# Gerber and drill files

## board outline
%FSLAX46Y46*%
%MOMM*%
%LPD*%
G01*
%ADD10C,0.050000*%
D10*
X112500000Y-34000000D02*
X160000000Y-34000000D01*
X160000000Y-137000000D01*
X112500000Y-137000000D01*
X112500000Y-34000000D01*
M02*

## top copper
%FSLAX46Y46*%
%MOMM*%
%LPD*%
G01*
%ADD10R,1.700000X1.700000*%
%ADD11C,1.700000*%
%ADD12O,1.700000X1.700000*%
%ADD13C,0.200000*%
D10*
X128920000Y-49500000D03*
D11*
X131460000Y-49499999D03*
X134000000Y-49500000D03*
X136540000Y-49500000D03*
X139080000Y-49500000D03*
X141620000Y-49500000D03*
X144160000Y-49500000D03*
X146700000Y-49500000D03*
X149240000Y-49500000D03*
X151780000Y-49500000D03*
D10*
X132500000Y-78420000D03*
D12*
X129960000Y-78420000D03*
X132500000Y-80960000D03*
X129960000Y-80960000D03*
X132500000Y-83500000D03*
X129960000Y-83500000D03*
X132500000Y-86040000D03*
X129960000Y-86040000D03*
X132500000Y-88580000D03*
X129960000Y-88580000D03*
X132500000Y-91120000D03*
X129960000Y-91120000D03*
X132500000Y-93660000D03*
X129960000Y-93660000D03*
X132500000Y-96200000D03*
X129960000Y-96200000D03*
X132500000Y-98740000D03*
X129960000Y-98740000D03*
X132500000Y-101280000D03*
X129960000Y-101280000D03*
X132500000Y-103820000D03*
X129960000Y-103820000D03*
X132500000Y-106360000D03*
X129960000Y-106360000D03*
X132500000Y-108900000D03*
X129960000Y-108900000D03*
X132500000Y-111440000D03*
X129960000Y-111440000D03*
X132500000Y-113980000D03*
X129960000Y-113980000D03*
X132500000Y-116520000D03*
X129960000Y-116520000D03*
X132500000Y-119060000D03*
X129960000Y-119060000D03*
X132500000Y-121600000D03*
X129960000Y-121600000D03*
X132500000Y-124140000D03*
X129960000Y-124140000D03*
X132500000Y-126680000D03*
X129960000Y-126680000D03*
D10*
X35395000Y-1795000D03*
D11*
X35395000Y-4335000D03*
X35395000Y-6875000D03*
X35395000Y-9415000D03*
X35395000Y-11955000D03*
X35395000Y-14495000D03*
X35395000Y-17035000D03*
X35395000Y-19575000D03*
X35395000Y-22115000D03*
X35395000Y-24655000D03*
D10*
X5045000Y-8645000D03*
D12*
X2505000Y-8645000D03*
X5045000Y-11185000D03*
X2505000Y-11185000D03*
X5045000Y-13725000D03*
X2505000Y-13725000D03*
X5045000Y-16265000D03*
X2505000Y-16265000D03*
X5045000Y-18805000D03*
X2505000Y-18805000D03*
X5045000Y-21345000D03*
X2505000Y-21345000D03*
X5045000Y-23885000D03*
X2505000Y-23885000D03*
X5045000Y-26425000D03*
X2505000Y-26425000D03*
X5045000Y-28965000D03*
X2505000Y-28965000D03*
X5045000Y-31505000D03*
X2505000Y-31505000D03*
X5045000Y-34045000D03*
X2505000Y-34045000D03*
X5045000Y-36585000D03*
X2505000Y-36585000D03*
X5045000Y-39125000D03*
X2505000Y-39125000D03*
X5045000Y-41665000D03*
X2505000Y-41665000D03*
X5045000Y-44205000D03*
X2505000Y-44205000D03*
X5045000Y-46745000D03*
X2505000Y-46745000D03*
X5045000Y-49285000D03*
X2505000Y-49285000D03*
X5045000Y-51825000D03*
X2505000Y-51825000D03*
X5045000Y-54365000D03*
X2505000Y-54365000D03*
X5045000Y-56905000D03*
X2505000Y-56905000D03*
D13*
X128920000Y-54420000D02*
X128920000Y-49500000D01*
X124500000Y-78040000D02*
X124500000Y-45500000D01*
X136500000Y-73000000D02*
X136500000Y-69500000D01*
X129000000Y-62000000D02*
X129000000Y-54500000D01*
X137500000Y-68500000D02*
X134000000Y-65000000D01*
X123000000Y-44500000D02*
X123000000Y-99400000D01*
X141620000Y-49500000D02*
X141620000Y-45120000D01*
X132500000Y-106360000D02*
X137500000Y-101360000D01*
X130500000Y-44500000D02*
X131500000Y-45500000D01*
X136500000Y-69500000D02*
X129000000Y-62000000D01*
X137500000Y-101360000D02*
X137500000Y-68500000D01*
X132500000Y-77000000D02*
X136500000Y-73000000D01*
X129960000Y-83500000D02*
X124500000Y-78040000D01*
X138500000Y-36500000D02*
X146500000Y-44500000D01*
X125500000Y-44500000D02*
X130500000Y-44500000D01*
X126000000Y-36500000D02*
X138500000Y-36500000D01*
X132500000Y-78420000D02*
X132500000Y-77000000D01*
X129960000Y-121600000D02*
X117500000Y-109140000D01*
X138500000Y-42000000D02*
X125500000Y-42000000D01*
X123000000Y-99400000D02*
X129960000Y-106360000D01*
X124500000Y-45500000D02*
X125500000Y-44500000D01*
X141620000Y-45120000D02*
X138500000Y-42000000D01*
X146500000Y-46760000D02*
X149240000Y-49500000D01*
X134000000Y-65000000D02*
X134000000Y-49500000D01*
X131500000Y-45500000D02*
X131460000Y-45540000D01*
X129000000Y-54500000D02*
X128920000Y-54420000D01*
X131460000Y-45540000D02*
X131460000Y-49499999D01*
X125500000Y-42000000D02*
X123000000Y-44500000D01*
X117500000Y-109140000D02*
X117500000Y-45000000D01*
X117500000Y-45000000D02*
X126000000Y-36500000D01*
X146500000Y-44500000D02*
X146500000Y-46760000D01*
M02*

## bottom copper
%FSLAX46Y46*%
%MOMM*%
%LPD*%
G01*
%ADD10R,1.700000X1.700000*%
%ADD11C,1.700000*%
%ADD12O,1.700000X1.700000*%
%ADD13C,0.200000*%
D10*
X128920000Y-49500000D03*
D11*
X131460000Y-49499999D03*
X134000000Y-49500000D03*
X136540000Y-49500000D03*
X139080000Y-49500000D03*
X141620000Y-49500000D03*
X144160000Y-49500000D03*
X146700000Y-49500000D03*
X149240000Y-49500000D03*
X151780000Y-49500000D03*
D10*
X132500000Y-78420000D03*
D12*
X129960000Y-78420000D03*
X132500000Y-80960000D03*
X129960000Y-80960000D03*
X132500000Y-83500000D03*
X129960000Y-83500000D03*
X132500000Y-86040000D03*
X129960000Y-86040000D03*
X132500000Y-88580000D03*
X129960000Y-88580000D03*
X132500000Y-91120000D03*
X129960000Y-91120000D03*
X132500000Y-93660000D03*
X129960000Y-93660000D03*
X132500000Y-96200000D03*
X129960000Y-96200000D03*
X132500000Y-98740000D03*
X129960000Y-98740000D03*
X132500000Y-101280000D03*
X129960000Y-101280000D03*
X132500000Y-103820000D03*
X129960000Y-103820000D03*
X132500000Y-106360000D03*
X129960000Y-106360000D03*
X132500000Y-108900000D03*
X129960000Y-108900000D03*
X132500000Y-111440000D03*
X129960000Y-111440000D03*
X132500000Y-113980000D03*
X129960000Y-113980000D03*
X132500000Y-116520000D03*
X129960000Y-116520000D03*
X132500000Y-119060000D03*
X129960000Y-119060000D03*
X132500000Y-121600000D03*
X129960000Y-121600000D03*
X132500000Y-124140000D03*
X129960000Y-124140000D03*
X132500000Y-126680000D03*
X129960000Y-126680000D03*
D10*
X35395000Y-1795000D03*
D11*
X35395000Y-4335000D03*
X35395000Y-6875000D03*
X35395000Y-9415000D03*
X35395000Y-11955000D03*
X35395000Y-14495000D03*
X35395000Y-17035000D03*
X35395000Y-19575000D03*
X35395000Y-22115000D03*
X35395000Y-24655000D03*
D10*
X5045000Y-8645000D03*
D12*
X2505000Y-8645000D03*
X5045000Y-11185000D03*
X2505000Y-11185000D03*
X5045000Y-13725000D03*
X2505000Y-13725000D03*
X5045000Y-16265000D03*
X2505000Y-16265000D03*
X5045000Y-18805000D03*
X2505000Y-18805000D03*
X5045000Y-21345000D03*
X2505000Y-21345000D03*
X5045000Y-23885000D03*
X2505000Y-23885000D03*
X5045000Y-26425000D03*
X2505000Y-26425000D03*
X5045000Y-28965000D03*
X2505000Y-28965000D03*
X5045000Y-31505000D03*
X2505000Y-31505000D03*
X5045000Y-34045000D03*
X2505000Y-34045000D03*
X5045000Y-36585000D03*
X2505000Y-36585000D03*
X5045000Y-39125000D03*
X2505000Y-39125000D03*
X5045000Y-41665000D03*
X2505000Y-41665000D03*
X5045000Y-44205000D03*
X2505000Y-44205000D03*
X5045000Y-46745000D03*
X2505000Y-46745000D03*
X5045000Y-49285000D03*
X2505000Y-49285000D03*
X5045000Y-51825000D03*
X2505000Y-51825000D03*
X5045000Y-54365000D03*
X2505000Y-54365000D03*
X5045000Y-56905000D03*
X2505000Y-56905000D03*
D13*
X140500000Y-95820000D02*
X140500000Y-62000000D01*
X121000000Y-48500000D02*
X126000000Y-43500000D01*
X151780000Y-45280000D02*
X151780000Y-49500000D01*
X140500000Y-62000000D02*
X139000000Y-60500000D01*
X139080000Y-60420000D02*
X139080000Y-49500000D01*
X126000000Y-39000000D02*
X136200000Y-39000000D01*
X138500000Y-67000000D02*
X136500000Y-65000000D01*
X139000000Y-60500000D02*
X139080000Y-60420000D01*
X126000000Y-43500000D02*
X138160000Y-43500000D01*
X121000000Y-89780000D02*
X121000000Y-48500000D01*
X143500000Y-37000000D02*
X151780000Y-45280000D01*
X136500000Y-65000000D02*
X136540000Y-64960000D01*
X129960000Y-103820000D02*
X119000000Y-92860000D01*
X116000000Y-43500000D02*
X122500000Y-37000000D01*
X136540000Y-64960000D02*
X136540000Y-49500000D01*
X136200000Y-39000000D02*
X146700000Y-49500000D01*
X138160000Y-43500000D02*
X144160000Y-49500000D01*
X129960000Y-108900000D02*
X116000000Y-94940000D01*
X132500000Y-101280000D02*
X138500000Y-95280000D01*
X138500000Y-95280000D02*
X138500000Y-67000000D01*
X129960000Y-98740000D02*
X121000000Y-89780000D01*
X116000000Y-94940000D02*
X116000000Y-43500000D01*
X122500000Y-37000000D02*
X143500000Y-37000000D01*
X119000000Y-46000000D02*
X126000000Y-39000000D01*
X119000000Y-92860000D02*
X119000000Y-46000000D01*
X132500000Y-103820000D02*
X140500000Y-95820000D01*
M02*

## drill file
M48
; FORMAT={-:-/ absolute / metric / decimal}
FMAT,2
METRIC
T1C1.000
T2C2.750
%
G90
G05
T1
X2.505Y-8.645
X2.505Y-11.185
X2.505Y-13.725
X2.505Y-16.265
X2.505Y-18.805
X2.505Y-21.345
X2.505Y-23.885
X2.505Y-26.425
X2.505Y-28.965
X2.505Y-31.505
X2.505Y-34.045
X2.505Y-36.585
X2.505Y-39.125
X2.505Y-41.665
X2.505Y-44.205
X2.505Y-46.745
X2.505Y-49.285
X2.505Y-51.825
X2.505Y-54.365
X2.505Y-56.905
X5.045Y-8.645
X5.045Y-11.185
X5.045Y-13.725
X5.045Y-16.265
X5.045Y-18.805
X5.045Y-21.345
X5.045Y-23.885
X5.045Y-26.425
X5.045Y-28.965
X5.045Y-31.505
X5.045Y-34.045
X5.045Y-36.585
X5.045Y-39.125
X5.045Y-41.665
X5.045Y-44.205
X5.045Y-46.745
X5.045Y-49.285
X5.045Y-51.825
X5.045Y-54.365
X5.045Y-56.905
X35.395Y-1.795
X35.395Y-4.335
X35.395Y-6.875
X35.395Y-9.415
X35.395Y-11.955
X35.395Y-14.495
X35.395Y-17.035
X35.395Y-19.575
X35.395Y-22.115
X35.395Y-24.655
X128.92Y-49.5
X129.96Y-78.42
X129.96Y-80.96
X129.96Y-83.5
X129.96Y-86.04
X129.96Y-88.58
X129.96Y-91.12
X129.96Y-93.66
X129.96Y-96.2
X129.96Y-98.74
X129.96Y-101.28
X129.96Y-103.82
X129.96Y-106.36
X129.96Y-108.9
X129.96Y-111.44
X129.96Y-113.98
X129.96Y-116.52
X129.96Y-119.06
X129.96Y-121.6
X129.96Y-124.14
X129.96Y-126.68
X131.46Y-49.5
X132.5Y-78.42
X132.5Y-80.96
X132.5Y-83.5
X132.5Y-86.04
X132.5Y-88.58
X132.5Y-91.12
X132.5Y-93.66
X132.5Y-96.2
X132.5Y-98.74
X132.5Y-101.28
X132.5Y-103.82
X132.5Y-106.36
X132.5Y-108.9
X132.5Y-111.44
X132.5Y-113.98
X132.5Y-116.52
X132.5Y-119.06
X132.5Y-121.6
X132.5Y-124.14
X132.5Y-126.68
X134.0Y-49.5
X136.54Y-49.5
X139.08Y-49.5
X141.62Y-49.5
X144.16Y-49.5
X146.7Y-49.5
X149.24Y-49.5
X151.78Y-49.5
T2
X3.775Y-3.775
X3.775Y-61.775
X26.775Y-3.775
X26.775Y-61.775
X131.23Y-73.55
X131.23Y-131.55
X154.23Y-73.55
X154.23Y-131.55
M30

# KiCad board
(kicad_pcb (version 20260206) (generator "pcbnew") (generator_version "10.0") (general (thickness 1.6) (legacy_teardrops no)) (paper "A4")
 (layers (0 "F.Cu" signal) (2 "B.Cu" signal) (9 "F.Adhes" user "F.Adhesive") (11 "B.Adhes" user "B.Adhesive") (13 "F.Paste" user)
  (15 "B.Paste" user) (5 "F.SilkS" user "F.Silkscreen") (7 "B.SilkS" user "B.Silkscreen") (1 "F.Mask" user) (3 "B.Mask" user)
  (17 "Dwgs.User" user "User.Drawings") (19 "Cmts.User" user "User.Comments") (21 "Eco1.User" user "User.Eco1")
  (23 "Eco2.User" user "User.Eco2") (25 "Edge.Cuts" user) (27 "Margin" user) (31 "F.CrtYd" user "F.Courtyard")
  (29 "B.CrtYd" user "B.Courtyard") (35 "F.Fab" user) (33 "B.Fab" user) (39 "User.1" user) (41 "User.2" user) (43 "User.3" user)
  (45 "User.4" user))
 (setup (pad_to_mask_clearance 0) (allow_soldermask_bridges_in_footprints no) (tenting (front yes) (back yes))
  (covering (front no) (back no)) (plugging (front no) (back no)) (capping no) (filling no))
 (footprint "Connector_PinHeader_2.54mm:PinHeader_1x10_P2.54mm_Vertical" (layer "F.Cu") (at 128.92 49.5 90)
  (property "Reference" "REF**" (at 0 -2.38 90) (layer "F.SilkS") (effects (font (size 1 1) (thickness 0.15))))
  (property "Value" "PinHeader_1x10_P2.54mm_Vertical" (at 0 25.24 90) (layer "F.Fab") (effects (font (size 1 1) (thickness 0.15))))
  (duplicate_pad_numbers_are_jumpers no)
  (pad "1" thru_hole rect (at 0 0 90) (size 1.7 1.7) (drill 1) (layers "*.Cu" "*.Mask") (remove_unused_layers no))
  (pad "2" thru_hole circle (at 0.000001 2.54 90) (size 1.7 1.7) (drill 1) (layers "*.Cu" "*.Mask") (remove_unused_layers no))
  (pad "3" thru_hole circle (at 0 5.08 90) (size 1.7 1.7) (drill 1) (layers "*.Cu" "*.Mask") (remove_unused_layers no))
  (pad "4" thru_hole circle (at 0 7.62 90) (size 1.7 1.7) (drill 1) (layers "*.Cu" "*.Mask") (remove_unused_layers no))
  (pad "5" thru_hole circle (at 0 10.16 90) (size 1.7 1.7) (drill 1) (layers "*.Cu" "*.Mask") (remove_unused_layers no))
  (pad "6" thru_hole circle (at 0 12.7 90) (size 1.7 1.7) (drill 1) (layers "*.Cu" "*.Mask") (remove_unused_layers no))
  (pad "7" thru_hole circle (at 0 15.24 90) (size 1.7 1.7) (drill 1) (layers "*.Cu" "*.Mask") (remove_unused_layers no))
  (pad "8" thru_hole circle (at 0 17.78 90) (size 1.7 1.7) (drill 1) (layers "*.Cu" "*.Mask") (remove_unused_layers no))
  (pad "9" thru_hole circle (at 0 20.32 90) (size 1.7 1.7) (drill 1) (layers "*.Cu" "*.Mask") (remove_unused_layers no))
  (pad "10" thru_hole circle (at 0 22.86 90) (size 1.7 1.7) (drill 1) (layers "*.Cu" "*.Mask") (remove_unused_layers no)))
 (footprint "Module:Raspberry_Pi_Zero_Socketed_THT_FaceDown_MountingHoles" (layer "F.Cu") (at 132.5 78.42)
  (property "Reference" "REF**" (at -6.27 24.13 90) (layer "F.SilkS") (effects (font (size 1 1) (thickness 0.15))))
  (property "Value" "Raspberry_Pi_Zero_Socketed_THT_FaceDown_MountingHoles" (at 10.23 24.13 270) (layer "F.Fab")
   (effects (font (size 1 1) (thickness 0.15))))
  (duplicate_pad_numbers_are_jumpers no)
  (pad "" np_thru_hole circle (at -1.27 -4.87 90) (size 2.75 2.75) (drill 2.75) (layers "*.Cu" "*.Mask") (solder_mask_margin 1.625))
  (pad "" np_thru_hole circle (at -1.27 53.13 90) (size 2.75 2.75) (drill 2.75) (layers "*.Cu" "*.Mask") (solder_mask_margin 1.625))
  (pad "" np_thru_hole circle (at 21.73 -4.87 90) (size 2.75 2.75) (drill 2.75) (layers "*.Cu" "*.Mask") (solder_mask_margin 1.625))
  (pad "" np_thru_hole circle (at 21.73 53.13 90) (size 2.75 2.75) (drill 2.75) (layers "*.Cu" "*.Mask") (solder_mask_margin 1.625))
  (pad "1" thru_hole rect (at 0 0) (size 1.7 1.7) (drill 1) (layers "*.Cu" "*.Mask") (remove_unused_layers no))
  (pad "2" thru_hole oval (at -2.54 0) (size 1.7 1.7) (drill 1) (layers "*.Cu" "*.Mask") (remove_unused_layers no))
  (pad "3" thru_hole oval (at 0 2.54) (size 1.7 1.7) (drill 1) (layers "*.Cu" "*.Mask") (remove_unused_layers no))
  (pad "4" thru_hole oval (at -2.54 2.54) (size 1.7 1.7) (drill 1) (layers "*.Cu" "*.Mask") (remove_unused_layers no))
  (pad "5" thru_hole oval (at 0 5.08) (size 1.7 1.7) (drill 1) (layers "*.Cu" "*.Mask") (remove_unused_layers no))
  (pad "6" thru_hole oval (at -2.54 5.08) (size 1.7 1.7) (drill 1) (layers "*.Cu" "*.Mask") (remove_unused_layers no))
  (pad "7" thru_hole oval (at 0 7.62) (size 1.7 1.7) (drill 1) (layers "*.Cu" "*.Mask") (remove_unused_layers no))
  (pad "8" thru_hole oval (at -2.54 7.62) (size 1.7 1.7) (drill 1) (layers "*.Cu" "*.Mask") (remove_unused_layers no))
  (pad "9" thru_hole oval (at 0 10.16) (size 1.7 1.7) (drill 1) (layers "*.Cu" "*.Mask") (remove_unused_layers no))
  (pad "10" thru_hole oval (at -2.54 10.16) (size 1.7 1.7) (drill 1) (layers "*.Cu" "*.Mask") (remove_unused_layers no))
  (pad "11" thru_hole oval (at 0 12.7) (size 1.7 1.7) (drill 1) (layers "*.Cu" "*.Mask") (remove_unused_layers no))
  (pad "12" thru_hole oval (at -2.54 12.7) (size 1.7 1.7) (drill 1) (layers "*.Cu" "*.Mask") (remove_unused_layers no))
  (pad "13" thru_hole oval (at 0 15.24) (size 1.7 1.7) (drill 1) (layers "*.Cu" "*.Mask") (remove_unused_layers no))
  (pad "14" thru_hole oval (at -2.54 15.24) (size 1.7 1.7) (drill 1) (layers "*.Cu" "*.Mask") (remove_unused_layers no))
  (pad "15" thru_hole oval (at 0 17.78) (size 1.7 1.7) (drill 1) (layers "*.Cu" "*.Mask") (remove_unused_layers no))
  (pad "16" thru_hole oval (at -2.54 17.78) (size 1.7 1.7) (drill 1) (layers "*.Cu" "*.Mask") (remove_unused_layers no))
  (pad "17" thru_hole oval (at 0 20.32) (size 1.7 1.7) (drill 1) (layers "*.Cu" "*.Mask") (remove_unused_layers no))
  (pad "18" thru_hole oval (at -2.54 20.32) (size 1.7 1.7) (drill 1) (layers "*.Cu" "*.Mask") (remove_unused_layers no))
  (pad "19" thru_hole oval (at 0 22.86) (size 1.7 1.7) (drill 1) (layers "*.Cu" "*.Mask") (remove_unused_layers no))
  (pad "20" thru_hole oval (at -2.54 22.86) (size 1.7 1.7) (drill 1) (layers "*.Cu" "*.Mask") (remove_unused_layers no))
  (pad "21" thru_hole oval (at 0 25.4) (size 1.7 1.7) (drill 1) (layers "*.Cu" "*.Mask") (remove_unused_layers no))
  (pad "22" thru_hole oval (at -2.54 25.4) (size 1.7 1.7) (drill 1) (layers "*.Cu" "*.Mask") (remove_unused_layers no))
  (pad "23" thru_hole oval (at 0 27.94) (size 1.7 1.7) (drill 1) (layers "*.Cu" "*.Mask") (remove_unused_layers no))
  (pad "24" thru_hole oval (at -2.54 27.94) (size 1.7 1.7) (drill 1) (layers "*.Cu" "*.Mask") (remove_unused_layers no))
  (pad "25" thru_hole oval (at 0 30.48) (size 1.7 1.7) (drill 1) (layers "*.Cu" "*.Mask") (remove_unused_layers no))
  (pad "26" thru_hole oval (at -2.54 30.48) (size 1.7 1.7) (drill 1) (layers "*.Cu" "*.Mask") (remove_unused_layers no))
  (pad "27" thru_hole oval (at 0 33.02) (size 1.7 1.7) (drill 1) (layers "*.Cu" "*.Mask") (remove_unused_layers no))
  (pad "28" thru_hole oval (at -2.54 33.02) (size 1.7 1.7) (drill 1) (layers "*.Cu" "*.Mask") (remove_unused_layers no))
  (pad "29" thru_hole oval (at 0 35.56) (size 1.7 1.7) (drill 1) (layers "*.Cu" "*.Mask") (remove_unused_layers no))
  (pad "30" thru_hole oval (at -2.54 35.56) (size 1.7 1.7) (drill 1) (layers "*.Cu" "*.Mask") (remove_unused_layers no))
  (pad "31" thru_hole oval (at 0 38.1) (size 1.7 1.7) (drill 1) (layers "*.Cu" "*.Mask") (remove_unused_layers no))
  (pad "32" thru_hole oval (at -2.54 38.1) (size 1.7 1.7) (drill 1) (layers "*.Cu" "*.Mask") (remove_unused_layers no))
  (pad "33" thru_hole oval (at 0 40.64) (size 1.7 1.7) (drill 1) (layers "*.Cu" "*.Mask") (remove_unused_layers no))
  (pad "34" thru_hole oval (at -2.54 40.64) (size 1.7 1.7) (drill 1) (layers "*.Cu" "*.Mask") (remove_unused_layers no))
  (pad "35" thru_hole oval (at 0 43.18) (size 1.7 1.7) (drill 1) (layers "*.Cu" "*.Mask") (remove_unused_layers no))
  (pad "36" thru_hole oval (at -2.54 43.18) (size 1.7 1.7) (drill 1) (layers "*.Cu" "*.Mask") (remove_unused_layers no))
  (pad "37" thru_hole oval (at 0 45.72) (size 1.7 1.7) (drill 1) (layers "*.Cu" "*.Mask") (remove_unused_layers no))
  (pad "38" thru_hole oval (at -2.54 45.72) (size 1.7 1.7) (drill 1) (layers "*.Cu" "*.Mask") (remove_unused_layers no))
  (pad "39" thru_hole oval (at 0 48.26) (size 1.7 1.7) (drill 1) (layers "*.Cu" "*.Mask") (remove_unused_layers no))
  (pad "40" thru_hole oval (at -2.54 48.26) (size 1.7 1.7) (drill 1) (layers "*.Cu" "*.Mask") (remove_unused_layers no)))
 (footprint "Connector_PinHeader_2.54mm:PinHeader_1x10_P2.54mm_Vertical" (layer "F.Cu") (at 35.395 1.795)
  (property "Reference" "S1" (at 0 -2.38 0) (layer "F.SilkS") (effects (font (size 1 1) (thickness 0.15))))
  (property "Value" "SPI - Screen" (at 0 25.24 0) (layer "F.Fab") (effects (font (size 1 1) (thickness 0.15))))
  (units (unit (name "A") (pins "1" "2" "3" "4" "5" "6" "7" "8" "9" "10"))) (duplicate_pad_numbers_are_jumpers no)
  (pad "1" thru_hole rect (at 0 0) (size 1.7 1.7) (drill 1) (layers "*.Cu" "*.Mask") (remove_unused_layers no) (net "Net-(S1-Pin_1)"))
  (pad "2" thru_hole circle (at 0 2.54) (size 1.7 1.7) (drill 1) (layers "*.Cu" "*.Mask") (remove_unused_layers no) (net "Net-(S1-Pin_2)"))
  (pad "3" thru_hole circle (at 0 5.08) (size 1.7 1.7) (drill 1) (layers "*.Cu" "*.Mask") (remove_unused_layers no)
   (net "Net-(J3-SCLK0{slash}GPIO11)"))
  (pad "4" thru_hole circle (at 0 7.62) (size 1.7 1.7) (drill 1) (layers "*.Cu" "*.Mask") (remove_unused_layers no)
   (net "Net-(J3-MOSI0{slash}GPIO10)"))
  (pad "5" thru_hole circle (at 0 10.16) (size 1.7 1.7) (drill 1) (layers "*.Cu" "*.Mask") (remove_unused_layers no)
   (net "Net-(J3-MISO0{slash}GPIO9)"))
  (pad "6" thru_hole circle (at 0 12.7) (size 1.7 1.7) (drill 1) (layers "*.Cu" "*.Mask") (remove_unused_layers no)
   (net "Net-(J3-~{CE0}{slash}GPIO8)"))
  (pad "7" thru_hole circle (at 0 15.24) (size 1.7 1.7) (drill 1) (layers "*.Cu" "*.Mask") (remove_unused_layers no) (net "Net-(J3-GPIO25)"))
  (pad "8" thru_hole circle (at 0 17.78) (size 1.7 1.7) (drill 1) (layers "*.Cu" "*.Mask") (remove_unused_layers no) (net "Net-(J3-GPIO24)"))
  (pad "9" thru_hole circle (at 0 20.32) (size 1.7 1.7) (drill 1) (layers "*.Cu" "*.Mask") (remove_unused_layers no)
   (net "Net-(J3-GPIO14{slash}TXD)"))
  (pad "10" thru_hole circle (at 0 22.86) (size 1.7 1.7) (drill 1) (layers "*.Cu" "*.Mask") (remove_unused_layers no)
   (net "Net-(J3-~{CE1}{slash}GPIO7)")))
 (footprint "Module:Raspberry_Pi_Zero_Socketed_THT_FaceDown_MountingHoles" (layer "F.Cu") (at 5.045 8.645)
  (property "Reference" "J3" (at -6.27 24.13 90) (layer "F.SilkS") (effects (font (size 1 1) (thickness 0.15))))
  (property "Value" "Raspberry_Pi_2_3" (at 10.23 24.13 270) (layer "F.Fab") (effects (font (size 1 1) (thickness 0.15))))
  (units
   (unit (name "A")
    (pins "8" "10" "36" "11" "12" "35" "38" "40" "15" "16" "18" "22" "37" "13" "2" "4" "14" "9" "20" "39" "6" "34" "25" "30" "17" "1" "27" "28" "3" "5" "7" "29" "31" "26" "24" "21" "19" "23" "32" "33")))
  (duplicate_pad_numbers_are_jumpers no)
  (pad "" np_thru_hole circle (at -1.27 -4.87 90) (size 2.75 2.75) (drill 2.75) (layers "*.Cu" "*.Mask") (solder_mask_margin 1.625))
  (pad "" np_thru_hole circle (at -1.27 53.13 90) (size 2.75 2.75) (drill 2.75) (layers "*.Cu" "*.Mask") (solder_mask_margin 1.625))
  (pad "" np_thru_hole circle (at 21.73 -4.87 90) (size 2.75 2.75) (drill 2.75) (layers "*.Cu" "*.Mask") (solder_mask_margin 1.625))
  (pad "" np_thru_hole circle (at 21.73 53.13 90) (size 2.75 2.75) (drill 2.75) (layers "*.Cu" "*.Mask") (solder_mask_margin 1.625))
  (pad "1" thru_hole rect (at 0 0) (size 1.7 1.7) (drill 1) (layers "*.Cu" "*.Mask") (remove_unused_layers no) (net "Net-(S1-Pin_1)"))
  (pad "2" thru_hole oval (at -2.54 0) (size 1.7 1.7) (drill 1) (layers "*.Cu" "*.Mask") (remove_unused_layers no) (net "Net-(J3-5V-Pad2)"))
  (pad "3" thru_hole oval (at 0 2.54) (size 1.7 1.7) (drill 1) (layers "*.Cu" "*.Mask") (remove_unused_layers no)
   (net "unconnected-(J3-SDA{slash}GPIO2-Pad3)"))
  (pad "4" thru_hole oval (at -2.54 2.54) (size 1.7 1.7) (drill 1) (layers "*.Cu" "*.Mask") (remove_unused_layers no)
   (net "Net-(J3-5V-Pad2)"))
  (pad "5" thru_hole oval (at 0 5.08) (size 1.7 1.7) (drill 1) (layers "*.Cu" "*.Mask") (remove_unused_layers no)
   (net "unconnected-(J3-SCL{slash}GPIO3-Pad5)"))
  (pad "6" thru_hole oval (at -2.54 5.08) (size 1.7 1.7) (drill 1) (layers "*.Cu" "*.Mask") (remove_unused_layers no) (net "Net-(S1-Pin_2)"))
  (pad "7" thru_hole oval (at 0 7.62) (size 1.7 1.7) (drill 1) (layers "*.Cu" "*.Mask") (remove_unused_layers no)
   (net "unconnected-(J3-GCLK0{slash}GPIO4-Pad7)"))
  (pad "8" thru_hole oval (at -2.54 7.62) (size 1.7 1.7) (drill 1) (layers "*.Cu" "*.Mask") (remove_unused_layers no)
   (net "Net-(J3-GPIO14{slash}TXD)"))
  (pad "9" thru_hole oval (at 0 10.16) (size 1.7 1.7) (drill 1) (layers "*.Cu" "*.Mask") (remove_unused_layers no) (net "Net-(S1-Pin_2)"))
  (pad "10" thru_hole oval (at -2.54 10.16) (size 1.7 1.7) (drill 1) (layers "*.Cu" "*.Mask") (remove_unused_layers no)
   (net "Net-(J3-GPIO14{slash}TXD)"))
  (pad "11" thru_hole oval (at 0 12.7) (size 1.7 1.7) (drill 1) (layers "*.Cu" "*.Mask") (remove_unused_layers no)
   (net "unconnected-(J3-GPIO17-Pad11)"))
  (pad "12" thru_hole oval (at -2.54 12.7) (size 1.7 1.7) (drill 1) (layers "*.Cu" "*.Mask") (remove_unused_layers no)
   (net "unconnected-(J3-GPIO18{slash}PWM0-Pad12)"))
  (pad "13" thru_hole oval (at 0 15.24) (size 1.7 1.7) (drill 1) (layers "*.Cu" "*.Mask") (remove_unused_layers no)
   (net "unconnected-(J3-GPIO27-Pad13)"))
  (pad "14" thru_hole oval (at -2.54 15.24) (size 1.7 1.7) (drill 1) (layers "*.Cu" "*.Mask") (remove_unused_layers no)
   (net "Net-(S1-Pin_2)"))
  (pad "15" thru_hole oval (at 0 17.78) (size 1.7 1.7) (drill 1) (layers "*.Cu" "*.Mask") (remove_unused_layers no)
   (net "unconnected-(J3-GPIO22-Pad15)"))
  (pad "16" thru_hole oval (at -2.54 17.78) (size 1.7 1.7) (drill 1) (layers "*.Cu" "*.Mask") (remove_unused_layers no)
   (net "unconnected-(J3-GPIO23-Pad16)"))
  (pad "17" thru_hole oval (at 0 20.32) (size 1.7 1.7) (drill 1) (layers "*.Cu" "*.Mask") (remove_unused_layers no) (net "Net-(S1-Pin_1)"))
  (pad "18" thru_hole oval (at -2.54 20.32) (size 1.7 1.7) (drill 1) (layers "*.Cu" "*.Mask") (remove_unused_layers no)
   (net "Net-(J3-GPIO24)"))
  (pad "19" thru_hole oval (at 0 22.86) (size 1.7 1.7) (drill 1) (layers "*.Cu" "*.Mask") (remove_unused_layers no)
   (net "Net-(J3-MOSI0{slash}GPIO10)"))
  (pad "20" thru_hole oval (at -2.54 22.86) (size 1.7 1.7) (drill 1) (layers "*.Cu" "*.Mask") (remove_unused_layers no)
   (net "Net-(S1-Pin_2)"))
  (pad "21" thru_hole oval (at 0 25.4) (size 1.7 1.7) (drill 1) (layers "*.Cu" "*.Mask") (remove_unused_layers no)
   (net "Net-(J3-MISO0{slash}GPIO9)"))
  (pad "22" thru_hole oval (at -2.54 25.4) (size 1.7 1.7) (drill 1) (layers "*.Cu" "*.Mask") (remove_unused_layers no)
   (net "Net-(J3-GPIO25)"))
  (pad "23" thru_hole oval (at 0 27.94) (size 1.7 1.7) (drill 1) (layers "*.Cu" "*.Mask") (remove_unused_layers no)
   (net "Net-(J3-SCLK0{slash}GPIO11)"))
  (pad "24" thru_hole oval (at -2.54 27.94) (size 1.7 1.7) (drill 1) (layers "*.Cu" "*.Mask") (remove_unused_layers no)
   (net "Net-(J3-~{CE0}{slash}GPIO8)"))
  (pad "25" thru_hole oval (at 0 30.48) (size 1.7 1.7) (drill 1) (layers "*.Cu" "*.Mask") (remove_unused_layers no) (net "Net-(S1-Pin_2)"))
  (pad "26" thru_hole oval (at -2.54 30.48) (size 1.7 1.7) (drill 1) (layers "*.Cu" "*.Mask") (remove_unused_layers no)
   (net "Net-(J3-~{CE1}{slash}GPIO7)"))
  (pad "27" thru_hole oval (at 0 33.02) (size 1.7 1.7) (drill 1) (layers "*.Cu" "*.Mask") (remove_unused_layers no)
   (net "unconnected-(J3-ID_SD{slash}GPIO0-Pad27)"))
  (pad "28" thru_hole oval (at -2.54 33.02) (size 1.7 1.7) (drill 1) (layers "*.Cu" "*.Mask") (remove_unused_layers no)
   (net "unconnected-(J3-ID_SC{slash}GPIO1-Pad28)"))
  (pad "29" thru_hole oval (at 0 35.56) (size 1.7 1.7) (drill 1) (layers "*.Cu" "*.Mask") (remove_unused_layers no)
   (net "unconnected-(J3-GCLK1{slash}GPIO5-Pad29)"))
  (pad "30" thru_hole oval (at -2.54 35.56) (size 1.7 1.7) (drill 1) (layers "*.Cu" "*.Mask") (remove_unused_layers no)
   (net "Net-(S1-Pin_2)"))
  (pad "31" thru_hole oval (at 0 38.1) (size 1.7 1.7) (drill 1) (layers "*.Cu" "*.Mask") (remove_unused_layers no)
   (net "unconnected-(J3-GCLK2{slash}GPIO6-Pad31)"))
  (pad "32" thru_hole oval (at -2.54 38.1) (size 1.7 1.7) (drill 1) (layers "*.Cu" "*.Mask") (remove_unused_layers no)
   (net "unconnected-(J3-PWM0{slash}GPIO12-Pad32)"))
  (pad "33" thru_hole oval (at 0 40.64) (size 1.7 1.7) (drill 1) (layers "*.Cu" "*.Mask") (remove_unused_layers no)
   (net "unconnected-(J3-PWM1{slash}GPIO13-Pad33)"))
  (pad "34" thru_hole oval (at -2.54 40.64) (size 1.7 1.7) (drill 1) (layers "*.Cu" "*.Mask") (remove_unused_layers no)
   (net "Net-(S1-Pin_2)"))
  (pad "35" thru_hole oval (at 0 43.18) (size 1.7 1.7) (drill 1) (layers "*.Cu" "*.Mask") (remove_unused_layers no)
   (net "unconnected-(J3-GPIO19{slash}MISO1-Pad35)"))
  (pad "36" thru_hole oval (at -2.54 43.18) (size 1.7 1.7) (drill 1) (layers "*.Cu" "*.Mask") (remove_unused_layers no)
   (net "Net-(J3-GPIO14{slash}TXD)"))
  (pad "37" thru_hole oval (at 0 45.72) (size 1.7 1.7) (drill 1) (layers "*.Cu" "*.Mask") (remove_unused_layers no)
   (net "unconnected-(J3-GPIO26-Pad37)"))
  (pad "38" thru_hole oval (at -2.54 45.72) (size 1.7 1.7) (drill 1) (layers "*.Cu" "*.Mask") (remove_unused_layers no)
   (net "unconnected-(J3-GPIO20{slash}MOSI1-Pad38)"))
  (pad "39" thru_hole oval (at 0 48.26) (size 1.7 1.7) (drill 1) (layers "*.Cu" "*.Mask") (remove_unused_layers no) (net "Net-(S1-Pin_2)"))
  (pad "40" thru_hole oval (at -2.54 48.26) (size 1.7 1.7) (drill 1) (layers "*.Cu" "*.Mask") (remove_unused_layers no)
   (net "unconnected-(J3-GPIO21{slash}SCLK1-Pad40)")))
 (gr_rect (start 112.5 34) (end 160 137) (stroke (width 0.05) (type default)) (fill no) (layer "Edge.Cuts"))
 (segment (start 128.92 54.42) (end 128.92 49.5) (width 0.2) (layer "F.Cu") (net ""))
 (segment (start 124.5 78.04) (end 124.5 45.5) (width 0.2) (layer "F.Cu") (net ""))
 (segment (start 136.5 73) (end 136.5 69.5) (width 0.2) (layer "F.Cu") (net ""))
 (segment (start 129 62) (end 129 54.5) (width 0.2) (layer "F.Cu") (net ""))
 (segment (start 137.5 68.5) (end 134 65) (width 0.2) (layer "F.Cu") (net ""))
 (segment (start 123 44.5) (end 123 99.4) (width 0.2) (layer "F.Cu") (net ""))
 (segment (start 141.62 49.5) (end 141.62 45.12) (width 0.2) (layer "F.Cu") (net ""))
 (segment (start 132.5 106.36) (end 137.5 101.36) (width 0.2) (layer "F.Cu") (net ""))
 (segment (start 130.5 44.5) (end 131.5 45.5) (width 0.2) (layer "F.Cu") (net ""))
 (segment (start 136.5 69.5) (end 129 62) (width 0.2) (layer "F.Cu") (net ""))
 (segment (start 137.5 101.36) (end 137.5 68.5) (width 0.2) (layer "F.Cu") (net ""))
 (segment (start 132.5 77) (end 136.5 73) (width 0.2) (layer "F.Cu") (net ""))
 (segment (start 129.96 83.5) (end 124.5 78.04) (width 0.2) (layer "F.Cu") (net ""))
 (segment (start 138.5 36.5) (end 146.5 44.5) (width 0.2) (layer "F.Cu") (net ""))
 (segment (start 125.5 44.5) (end 130.5 44.5) (width 0.2) (layer "F.Cu") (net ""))
 (segment (start 126 36.5) (end 138.5 36.5) (width 0.2) (layer "F.Cu") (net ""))
 (segment (start 132.5 78.42) (end 132.5 77) (width 0.2) (layer "F.Cu") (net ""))
 (segment (start 129.96 121.6) (end 117.5 109.14) (width 0.2) (layer "F.Cu") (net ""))
 (segment (start 138.5 42) (end 125.5 42) (width 0.2) (layer "F.Cu") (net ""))
 (segment (start 123 99.4) (end 129.96 106.36) (width 0.2) (layer "F.Cu") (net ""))
 (segment (start 124.5 45.5) (end 125.5 44.5) (width 0.2) (layer "F.Cu") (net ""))
 (segment (start 141.62 45.12) (end 138.5 42) (width 0.2) (layer "F.Cu") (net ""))
 (segment (start 146.5 46.76) (end 149.24 49.5) (width 0.2) (layer "F.Cu") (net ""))
 (segment (start 134 65) (end 134 49.5) (width 0.2) (layer "F.Cu") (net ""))
 (segment (start 131.5 45.5) (end 131.46 45.54) (width 0.2) (layer "F.Cu") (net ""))
 (segment (start 129 54.5) (end 128.92 54.42) (width 0.2) (layer "F.Cu") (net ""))
 (segment (start 131.46 45.54) (end 131.46 49.499999) (width 0.2) (layer "F.Cu") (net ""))
 (segment (start 125.5 42) (end 123 44.5) (width 0.2) (layer "F.Cu") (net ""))
 (segment (start 117.5 109.14) (end 117.5 45) (width 0.2) (layer "F.Cu") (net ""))
 (segment (start 117.5 45) (end 126 36.5) (width 0.2) (layer "F.Cu") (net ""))
 (segment (start 146.5 44.5) (end 146.5 46.76) (width 0.2) (layer "F.Cu") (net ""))
 (segment (start 140.5 95.82) (end 140.5 62) (width 0.2) (layer "B.Cu") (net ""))
 (segment (start 121 48.5) (end 126 43.5) (width 0.2) (layer "B.Cu") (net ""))
 (segment (start 151.78 45.28) (end 151.78 49.5) (width 0.2) (layer "B.Cu") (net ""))
 (segment (start 140.5 62) (end 139 60.5) (width 0.2) (layer "B.Cu") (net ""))
 (segment (start 139.08 60.42) (end 139.08 49.5) (width 0.2) (layer "B.Cu") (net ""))
 (segment (start 126 39) (end 136.2 39) (width 0.2) (layer "B.Cu") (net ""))
 (segment (start 138.5 67) (end 136.5 65) (width 0.2) (layer "B.Cu") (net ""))
 (segment (start 139 60.5) (end 139.08 60.42) (width 0.2) (layer "B.Cu") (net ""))
 (segment (start 126 43.5) (end 138.16 43.5) (width 0.2) (layer "B.Cu") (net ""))
 (segment (start 121 89.78) (end 121 48.5) (width 0.2) (layer "B.Cu") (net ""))
 (segment (start 143.5 37) (end 151.78 45.28) (width 0.2) (layer "B.Cu") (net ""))
 (segment (start 136.5 65) (end 136.54 64.96) (width 0.2) (layer "B.Cu") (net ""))
 (segment (start 129.96 103.82) (end 119 92.86) (width 0.2) (layer "B.Cu") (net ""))
 (segment (start 116 43.5) (end 122.5 37) (width 0.2) (layer "B.Cu") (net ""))
 (segment (start 136.54 64.96) (end 136.54 49.5) (width 0.2) (layer "B.Cu") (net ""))
 (segment (start 136.2 39) (end 146.7 49.5) (width 0.2) (layer "B.Cu") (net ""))
 (segment (start 138.16 43.5) (end 144.16 49.5) (width 0.2) (layer "B.Cu") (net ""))
 (segment (start 129.96 108.9) (end 116 94.94) (width 0.2) (layer "B.Cu") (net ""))
 (segment (start 132.5 101.28) (end 138.5 95.28) (width 0.2) (layer "B.Cu") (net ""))
 (segment (start 138.5 95.28) (end 138.5 67) (width 0.2) (layer "B.Cu") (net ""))
 (segment (start 129.96 98.74) (end 121 89.78) (width 0.2) (layer "B.Cu") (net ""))
 (segment (start 116 94.94) (end 116 43.5) (width 0.2) (layer "B.Cu") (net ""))
 (segment (start 122.5 37) (end 143.5 37) (width 0.2) (layer "B.Cu") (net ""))
 (segment (start 119 46) (end 126 39) (width 0.2) (layer "B.Cu") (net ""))
 (segment (start 119 92.86) (end 119 46) (width 0.2) (layer "B.Cu") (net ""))
 (segment (start 132.5 103.82) (end 140.5 95.82) (width 0.2) (layer "B.Cu") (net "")))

